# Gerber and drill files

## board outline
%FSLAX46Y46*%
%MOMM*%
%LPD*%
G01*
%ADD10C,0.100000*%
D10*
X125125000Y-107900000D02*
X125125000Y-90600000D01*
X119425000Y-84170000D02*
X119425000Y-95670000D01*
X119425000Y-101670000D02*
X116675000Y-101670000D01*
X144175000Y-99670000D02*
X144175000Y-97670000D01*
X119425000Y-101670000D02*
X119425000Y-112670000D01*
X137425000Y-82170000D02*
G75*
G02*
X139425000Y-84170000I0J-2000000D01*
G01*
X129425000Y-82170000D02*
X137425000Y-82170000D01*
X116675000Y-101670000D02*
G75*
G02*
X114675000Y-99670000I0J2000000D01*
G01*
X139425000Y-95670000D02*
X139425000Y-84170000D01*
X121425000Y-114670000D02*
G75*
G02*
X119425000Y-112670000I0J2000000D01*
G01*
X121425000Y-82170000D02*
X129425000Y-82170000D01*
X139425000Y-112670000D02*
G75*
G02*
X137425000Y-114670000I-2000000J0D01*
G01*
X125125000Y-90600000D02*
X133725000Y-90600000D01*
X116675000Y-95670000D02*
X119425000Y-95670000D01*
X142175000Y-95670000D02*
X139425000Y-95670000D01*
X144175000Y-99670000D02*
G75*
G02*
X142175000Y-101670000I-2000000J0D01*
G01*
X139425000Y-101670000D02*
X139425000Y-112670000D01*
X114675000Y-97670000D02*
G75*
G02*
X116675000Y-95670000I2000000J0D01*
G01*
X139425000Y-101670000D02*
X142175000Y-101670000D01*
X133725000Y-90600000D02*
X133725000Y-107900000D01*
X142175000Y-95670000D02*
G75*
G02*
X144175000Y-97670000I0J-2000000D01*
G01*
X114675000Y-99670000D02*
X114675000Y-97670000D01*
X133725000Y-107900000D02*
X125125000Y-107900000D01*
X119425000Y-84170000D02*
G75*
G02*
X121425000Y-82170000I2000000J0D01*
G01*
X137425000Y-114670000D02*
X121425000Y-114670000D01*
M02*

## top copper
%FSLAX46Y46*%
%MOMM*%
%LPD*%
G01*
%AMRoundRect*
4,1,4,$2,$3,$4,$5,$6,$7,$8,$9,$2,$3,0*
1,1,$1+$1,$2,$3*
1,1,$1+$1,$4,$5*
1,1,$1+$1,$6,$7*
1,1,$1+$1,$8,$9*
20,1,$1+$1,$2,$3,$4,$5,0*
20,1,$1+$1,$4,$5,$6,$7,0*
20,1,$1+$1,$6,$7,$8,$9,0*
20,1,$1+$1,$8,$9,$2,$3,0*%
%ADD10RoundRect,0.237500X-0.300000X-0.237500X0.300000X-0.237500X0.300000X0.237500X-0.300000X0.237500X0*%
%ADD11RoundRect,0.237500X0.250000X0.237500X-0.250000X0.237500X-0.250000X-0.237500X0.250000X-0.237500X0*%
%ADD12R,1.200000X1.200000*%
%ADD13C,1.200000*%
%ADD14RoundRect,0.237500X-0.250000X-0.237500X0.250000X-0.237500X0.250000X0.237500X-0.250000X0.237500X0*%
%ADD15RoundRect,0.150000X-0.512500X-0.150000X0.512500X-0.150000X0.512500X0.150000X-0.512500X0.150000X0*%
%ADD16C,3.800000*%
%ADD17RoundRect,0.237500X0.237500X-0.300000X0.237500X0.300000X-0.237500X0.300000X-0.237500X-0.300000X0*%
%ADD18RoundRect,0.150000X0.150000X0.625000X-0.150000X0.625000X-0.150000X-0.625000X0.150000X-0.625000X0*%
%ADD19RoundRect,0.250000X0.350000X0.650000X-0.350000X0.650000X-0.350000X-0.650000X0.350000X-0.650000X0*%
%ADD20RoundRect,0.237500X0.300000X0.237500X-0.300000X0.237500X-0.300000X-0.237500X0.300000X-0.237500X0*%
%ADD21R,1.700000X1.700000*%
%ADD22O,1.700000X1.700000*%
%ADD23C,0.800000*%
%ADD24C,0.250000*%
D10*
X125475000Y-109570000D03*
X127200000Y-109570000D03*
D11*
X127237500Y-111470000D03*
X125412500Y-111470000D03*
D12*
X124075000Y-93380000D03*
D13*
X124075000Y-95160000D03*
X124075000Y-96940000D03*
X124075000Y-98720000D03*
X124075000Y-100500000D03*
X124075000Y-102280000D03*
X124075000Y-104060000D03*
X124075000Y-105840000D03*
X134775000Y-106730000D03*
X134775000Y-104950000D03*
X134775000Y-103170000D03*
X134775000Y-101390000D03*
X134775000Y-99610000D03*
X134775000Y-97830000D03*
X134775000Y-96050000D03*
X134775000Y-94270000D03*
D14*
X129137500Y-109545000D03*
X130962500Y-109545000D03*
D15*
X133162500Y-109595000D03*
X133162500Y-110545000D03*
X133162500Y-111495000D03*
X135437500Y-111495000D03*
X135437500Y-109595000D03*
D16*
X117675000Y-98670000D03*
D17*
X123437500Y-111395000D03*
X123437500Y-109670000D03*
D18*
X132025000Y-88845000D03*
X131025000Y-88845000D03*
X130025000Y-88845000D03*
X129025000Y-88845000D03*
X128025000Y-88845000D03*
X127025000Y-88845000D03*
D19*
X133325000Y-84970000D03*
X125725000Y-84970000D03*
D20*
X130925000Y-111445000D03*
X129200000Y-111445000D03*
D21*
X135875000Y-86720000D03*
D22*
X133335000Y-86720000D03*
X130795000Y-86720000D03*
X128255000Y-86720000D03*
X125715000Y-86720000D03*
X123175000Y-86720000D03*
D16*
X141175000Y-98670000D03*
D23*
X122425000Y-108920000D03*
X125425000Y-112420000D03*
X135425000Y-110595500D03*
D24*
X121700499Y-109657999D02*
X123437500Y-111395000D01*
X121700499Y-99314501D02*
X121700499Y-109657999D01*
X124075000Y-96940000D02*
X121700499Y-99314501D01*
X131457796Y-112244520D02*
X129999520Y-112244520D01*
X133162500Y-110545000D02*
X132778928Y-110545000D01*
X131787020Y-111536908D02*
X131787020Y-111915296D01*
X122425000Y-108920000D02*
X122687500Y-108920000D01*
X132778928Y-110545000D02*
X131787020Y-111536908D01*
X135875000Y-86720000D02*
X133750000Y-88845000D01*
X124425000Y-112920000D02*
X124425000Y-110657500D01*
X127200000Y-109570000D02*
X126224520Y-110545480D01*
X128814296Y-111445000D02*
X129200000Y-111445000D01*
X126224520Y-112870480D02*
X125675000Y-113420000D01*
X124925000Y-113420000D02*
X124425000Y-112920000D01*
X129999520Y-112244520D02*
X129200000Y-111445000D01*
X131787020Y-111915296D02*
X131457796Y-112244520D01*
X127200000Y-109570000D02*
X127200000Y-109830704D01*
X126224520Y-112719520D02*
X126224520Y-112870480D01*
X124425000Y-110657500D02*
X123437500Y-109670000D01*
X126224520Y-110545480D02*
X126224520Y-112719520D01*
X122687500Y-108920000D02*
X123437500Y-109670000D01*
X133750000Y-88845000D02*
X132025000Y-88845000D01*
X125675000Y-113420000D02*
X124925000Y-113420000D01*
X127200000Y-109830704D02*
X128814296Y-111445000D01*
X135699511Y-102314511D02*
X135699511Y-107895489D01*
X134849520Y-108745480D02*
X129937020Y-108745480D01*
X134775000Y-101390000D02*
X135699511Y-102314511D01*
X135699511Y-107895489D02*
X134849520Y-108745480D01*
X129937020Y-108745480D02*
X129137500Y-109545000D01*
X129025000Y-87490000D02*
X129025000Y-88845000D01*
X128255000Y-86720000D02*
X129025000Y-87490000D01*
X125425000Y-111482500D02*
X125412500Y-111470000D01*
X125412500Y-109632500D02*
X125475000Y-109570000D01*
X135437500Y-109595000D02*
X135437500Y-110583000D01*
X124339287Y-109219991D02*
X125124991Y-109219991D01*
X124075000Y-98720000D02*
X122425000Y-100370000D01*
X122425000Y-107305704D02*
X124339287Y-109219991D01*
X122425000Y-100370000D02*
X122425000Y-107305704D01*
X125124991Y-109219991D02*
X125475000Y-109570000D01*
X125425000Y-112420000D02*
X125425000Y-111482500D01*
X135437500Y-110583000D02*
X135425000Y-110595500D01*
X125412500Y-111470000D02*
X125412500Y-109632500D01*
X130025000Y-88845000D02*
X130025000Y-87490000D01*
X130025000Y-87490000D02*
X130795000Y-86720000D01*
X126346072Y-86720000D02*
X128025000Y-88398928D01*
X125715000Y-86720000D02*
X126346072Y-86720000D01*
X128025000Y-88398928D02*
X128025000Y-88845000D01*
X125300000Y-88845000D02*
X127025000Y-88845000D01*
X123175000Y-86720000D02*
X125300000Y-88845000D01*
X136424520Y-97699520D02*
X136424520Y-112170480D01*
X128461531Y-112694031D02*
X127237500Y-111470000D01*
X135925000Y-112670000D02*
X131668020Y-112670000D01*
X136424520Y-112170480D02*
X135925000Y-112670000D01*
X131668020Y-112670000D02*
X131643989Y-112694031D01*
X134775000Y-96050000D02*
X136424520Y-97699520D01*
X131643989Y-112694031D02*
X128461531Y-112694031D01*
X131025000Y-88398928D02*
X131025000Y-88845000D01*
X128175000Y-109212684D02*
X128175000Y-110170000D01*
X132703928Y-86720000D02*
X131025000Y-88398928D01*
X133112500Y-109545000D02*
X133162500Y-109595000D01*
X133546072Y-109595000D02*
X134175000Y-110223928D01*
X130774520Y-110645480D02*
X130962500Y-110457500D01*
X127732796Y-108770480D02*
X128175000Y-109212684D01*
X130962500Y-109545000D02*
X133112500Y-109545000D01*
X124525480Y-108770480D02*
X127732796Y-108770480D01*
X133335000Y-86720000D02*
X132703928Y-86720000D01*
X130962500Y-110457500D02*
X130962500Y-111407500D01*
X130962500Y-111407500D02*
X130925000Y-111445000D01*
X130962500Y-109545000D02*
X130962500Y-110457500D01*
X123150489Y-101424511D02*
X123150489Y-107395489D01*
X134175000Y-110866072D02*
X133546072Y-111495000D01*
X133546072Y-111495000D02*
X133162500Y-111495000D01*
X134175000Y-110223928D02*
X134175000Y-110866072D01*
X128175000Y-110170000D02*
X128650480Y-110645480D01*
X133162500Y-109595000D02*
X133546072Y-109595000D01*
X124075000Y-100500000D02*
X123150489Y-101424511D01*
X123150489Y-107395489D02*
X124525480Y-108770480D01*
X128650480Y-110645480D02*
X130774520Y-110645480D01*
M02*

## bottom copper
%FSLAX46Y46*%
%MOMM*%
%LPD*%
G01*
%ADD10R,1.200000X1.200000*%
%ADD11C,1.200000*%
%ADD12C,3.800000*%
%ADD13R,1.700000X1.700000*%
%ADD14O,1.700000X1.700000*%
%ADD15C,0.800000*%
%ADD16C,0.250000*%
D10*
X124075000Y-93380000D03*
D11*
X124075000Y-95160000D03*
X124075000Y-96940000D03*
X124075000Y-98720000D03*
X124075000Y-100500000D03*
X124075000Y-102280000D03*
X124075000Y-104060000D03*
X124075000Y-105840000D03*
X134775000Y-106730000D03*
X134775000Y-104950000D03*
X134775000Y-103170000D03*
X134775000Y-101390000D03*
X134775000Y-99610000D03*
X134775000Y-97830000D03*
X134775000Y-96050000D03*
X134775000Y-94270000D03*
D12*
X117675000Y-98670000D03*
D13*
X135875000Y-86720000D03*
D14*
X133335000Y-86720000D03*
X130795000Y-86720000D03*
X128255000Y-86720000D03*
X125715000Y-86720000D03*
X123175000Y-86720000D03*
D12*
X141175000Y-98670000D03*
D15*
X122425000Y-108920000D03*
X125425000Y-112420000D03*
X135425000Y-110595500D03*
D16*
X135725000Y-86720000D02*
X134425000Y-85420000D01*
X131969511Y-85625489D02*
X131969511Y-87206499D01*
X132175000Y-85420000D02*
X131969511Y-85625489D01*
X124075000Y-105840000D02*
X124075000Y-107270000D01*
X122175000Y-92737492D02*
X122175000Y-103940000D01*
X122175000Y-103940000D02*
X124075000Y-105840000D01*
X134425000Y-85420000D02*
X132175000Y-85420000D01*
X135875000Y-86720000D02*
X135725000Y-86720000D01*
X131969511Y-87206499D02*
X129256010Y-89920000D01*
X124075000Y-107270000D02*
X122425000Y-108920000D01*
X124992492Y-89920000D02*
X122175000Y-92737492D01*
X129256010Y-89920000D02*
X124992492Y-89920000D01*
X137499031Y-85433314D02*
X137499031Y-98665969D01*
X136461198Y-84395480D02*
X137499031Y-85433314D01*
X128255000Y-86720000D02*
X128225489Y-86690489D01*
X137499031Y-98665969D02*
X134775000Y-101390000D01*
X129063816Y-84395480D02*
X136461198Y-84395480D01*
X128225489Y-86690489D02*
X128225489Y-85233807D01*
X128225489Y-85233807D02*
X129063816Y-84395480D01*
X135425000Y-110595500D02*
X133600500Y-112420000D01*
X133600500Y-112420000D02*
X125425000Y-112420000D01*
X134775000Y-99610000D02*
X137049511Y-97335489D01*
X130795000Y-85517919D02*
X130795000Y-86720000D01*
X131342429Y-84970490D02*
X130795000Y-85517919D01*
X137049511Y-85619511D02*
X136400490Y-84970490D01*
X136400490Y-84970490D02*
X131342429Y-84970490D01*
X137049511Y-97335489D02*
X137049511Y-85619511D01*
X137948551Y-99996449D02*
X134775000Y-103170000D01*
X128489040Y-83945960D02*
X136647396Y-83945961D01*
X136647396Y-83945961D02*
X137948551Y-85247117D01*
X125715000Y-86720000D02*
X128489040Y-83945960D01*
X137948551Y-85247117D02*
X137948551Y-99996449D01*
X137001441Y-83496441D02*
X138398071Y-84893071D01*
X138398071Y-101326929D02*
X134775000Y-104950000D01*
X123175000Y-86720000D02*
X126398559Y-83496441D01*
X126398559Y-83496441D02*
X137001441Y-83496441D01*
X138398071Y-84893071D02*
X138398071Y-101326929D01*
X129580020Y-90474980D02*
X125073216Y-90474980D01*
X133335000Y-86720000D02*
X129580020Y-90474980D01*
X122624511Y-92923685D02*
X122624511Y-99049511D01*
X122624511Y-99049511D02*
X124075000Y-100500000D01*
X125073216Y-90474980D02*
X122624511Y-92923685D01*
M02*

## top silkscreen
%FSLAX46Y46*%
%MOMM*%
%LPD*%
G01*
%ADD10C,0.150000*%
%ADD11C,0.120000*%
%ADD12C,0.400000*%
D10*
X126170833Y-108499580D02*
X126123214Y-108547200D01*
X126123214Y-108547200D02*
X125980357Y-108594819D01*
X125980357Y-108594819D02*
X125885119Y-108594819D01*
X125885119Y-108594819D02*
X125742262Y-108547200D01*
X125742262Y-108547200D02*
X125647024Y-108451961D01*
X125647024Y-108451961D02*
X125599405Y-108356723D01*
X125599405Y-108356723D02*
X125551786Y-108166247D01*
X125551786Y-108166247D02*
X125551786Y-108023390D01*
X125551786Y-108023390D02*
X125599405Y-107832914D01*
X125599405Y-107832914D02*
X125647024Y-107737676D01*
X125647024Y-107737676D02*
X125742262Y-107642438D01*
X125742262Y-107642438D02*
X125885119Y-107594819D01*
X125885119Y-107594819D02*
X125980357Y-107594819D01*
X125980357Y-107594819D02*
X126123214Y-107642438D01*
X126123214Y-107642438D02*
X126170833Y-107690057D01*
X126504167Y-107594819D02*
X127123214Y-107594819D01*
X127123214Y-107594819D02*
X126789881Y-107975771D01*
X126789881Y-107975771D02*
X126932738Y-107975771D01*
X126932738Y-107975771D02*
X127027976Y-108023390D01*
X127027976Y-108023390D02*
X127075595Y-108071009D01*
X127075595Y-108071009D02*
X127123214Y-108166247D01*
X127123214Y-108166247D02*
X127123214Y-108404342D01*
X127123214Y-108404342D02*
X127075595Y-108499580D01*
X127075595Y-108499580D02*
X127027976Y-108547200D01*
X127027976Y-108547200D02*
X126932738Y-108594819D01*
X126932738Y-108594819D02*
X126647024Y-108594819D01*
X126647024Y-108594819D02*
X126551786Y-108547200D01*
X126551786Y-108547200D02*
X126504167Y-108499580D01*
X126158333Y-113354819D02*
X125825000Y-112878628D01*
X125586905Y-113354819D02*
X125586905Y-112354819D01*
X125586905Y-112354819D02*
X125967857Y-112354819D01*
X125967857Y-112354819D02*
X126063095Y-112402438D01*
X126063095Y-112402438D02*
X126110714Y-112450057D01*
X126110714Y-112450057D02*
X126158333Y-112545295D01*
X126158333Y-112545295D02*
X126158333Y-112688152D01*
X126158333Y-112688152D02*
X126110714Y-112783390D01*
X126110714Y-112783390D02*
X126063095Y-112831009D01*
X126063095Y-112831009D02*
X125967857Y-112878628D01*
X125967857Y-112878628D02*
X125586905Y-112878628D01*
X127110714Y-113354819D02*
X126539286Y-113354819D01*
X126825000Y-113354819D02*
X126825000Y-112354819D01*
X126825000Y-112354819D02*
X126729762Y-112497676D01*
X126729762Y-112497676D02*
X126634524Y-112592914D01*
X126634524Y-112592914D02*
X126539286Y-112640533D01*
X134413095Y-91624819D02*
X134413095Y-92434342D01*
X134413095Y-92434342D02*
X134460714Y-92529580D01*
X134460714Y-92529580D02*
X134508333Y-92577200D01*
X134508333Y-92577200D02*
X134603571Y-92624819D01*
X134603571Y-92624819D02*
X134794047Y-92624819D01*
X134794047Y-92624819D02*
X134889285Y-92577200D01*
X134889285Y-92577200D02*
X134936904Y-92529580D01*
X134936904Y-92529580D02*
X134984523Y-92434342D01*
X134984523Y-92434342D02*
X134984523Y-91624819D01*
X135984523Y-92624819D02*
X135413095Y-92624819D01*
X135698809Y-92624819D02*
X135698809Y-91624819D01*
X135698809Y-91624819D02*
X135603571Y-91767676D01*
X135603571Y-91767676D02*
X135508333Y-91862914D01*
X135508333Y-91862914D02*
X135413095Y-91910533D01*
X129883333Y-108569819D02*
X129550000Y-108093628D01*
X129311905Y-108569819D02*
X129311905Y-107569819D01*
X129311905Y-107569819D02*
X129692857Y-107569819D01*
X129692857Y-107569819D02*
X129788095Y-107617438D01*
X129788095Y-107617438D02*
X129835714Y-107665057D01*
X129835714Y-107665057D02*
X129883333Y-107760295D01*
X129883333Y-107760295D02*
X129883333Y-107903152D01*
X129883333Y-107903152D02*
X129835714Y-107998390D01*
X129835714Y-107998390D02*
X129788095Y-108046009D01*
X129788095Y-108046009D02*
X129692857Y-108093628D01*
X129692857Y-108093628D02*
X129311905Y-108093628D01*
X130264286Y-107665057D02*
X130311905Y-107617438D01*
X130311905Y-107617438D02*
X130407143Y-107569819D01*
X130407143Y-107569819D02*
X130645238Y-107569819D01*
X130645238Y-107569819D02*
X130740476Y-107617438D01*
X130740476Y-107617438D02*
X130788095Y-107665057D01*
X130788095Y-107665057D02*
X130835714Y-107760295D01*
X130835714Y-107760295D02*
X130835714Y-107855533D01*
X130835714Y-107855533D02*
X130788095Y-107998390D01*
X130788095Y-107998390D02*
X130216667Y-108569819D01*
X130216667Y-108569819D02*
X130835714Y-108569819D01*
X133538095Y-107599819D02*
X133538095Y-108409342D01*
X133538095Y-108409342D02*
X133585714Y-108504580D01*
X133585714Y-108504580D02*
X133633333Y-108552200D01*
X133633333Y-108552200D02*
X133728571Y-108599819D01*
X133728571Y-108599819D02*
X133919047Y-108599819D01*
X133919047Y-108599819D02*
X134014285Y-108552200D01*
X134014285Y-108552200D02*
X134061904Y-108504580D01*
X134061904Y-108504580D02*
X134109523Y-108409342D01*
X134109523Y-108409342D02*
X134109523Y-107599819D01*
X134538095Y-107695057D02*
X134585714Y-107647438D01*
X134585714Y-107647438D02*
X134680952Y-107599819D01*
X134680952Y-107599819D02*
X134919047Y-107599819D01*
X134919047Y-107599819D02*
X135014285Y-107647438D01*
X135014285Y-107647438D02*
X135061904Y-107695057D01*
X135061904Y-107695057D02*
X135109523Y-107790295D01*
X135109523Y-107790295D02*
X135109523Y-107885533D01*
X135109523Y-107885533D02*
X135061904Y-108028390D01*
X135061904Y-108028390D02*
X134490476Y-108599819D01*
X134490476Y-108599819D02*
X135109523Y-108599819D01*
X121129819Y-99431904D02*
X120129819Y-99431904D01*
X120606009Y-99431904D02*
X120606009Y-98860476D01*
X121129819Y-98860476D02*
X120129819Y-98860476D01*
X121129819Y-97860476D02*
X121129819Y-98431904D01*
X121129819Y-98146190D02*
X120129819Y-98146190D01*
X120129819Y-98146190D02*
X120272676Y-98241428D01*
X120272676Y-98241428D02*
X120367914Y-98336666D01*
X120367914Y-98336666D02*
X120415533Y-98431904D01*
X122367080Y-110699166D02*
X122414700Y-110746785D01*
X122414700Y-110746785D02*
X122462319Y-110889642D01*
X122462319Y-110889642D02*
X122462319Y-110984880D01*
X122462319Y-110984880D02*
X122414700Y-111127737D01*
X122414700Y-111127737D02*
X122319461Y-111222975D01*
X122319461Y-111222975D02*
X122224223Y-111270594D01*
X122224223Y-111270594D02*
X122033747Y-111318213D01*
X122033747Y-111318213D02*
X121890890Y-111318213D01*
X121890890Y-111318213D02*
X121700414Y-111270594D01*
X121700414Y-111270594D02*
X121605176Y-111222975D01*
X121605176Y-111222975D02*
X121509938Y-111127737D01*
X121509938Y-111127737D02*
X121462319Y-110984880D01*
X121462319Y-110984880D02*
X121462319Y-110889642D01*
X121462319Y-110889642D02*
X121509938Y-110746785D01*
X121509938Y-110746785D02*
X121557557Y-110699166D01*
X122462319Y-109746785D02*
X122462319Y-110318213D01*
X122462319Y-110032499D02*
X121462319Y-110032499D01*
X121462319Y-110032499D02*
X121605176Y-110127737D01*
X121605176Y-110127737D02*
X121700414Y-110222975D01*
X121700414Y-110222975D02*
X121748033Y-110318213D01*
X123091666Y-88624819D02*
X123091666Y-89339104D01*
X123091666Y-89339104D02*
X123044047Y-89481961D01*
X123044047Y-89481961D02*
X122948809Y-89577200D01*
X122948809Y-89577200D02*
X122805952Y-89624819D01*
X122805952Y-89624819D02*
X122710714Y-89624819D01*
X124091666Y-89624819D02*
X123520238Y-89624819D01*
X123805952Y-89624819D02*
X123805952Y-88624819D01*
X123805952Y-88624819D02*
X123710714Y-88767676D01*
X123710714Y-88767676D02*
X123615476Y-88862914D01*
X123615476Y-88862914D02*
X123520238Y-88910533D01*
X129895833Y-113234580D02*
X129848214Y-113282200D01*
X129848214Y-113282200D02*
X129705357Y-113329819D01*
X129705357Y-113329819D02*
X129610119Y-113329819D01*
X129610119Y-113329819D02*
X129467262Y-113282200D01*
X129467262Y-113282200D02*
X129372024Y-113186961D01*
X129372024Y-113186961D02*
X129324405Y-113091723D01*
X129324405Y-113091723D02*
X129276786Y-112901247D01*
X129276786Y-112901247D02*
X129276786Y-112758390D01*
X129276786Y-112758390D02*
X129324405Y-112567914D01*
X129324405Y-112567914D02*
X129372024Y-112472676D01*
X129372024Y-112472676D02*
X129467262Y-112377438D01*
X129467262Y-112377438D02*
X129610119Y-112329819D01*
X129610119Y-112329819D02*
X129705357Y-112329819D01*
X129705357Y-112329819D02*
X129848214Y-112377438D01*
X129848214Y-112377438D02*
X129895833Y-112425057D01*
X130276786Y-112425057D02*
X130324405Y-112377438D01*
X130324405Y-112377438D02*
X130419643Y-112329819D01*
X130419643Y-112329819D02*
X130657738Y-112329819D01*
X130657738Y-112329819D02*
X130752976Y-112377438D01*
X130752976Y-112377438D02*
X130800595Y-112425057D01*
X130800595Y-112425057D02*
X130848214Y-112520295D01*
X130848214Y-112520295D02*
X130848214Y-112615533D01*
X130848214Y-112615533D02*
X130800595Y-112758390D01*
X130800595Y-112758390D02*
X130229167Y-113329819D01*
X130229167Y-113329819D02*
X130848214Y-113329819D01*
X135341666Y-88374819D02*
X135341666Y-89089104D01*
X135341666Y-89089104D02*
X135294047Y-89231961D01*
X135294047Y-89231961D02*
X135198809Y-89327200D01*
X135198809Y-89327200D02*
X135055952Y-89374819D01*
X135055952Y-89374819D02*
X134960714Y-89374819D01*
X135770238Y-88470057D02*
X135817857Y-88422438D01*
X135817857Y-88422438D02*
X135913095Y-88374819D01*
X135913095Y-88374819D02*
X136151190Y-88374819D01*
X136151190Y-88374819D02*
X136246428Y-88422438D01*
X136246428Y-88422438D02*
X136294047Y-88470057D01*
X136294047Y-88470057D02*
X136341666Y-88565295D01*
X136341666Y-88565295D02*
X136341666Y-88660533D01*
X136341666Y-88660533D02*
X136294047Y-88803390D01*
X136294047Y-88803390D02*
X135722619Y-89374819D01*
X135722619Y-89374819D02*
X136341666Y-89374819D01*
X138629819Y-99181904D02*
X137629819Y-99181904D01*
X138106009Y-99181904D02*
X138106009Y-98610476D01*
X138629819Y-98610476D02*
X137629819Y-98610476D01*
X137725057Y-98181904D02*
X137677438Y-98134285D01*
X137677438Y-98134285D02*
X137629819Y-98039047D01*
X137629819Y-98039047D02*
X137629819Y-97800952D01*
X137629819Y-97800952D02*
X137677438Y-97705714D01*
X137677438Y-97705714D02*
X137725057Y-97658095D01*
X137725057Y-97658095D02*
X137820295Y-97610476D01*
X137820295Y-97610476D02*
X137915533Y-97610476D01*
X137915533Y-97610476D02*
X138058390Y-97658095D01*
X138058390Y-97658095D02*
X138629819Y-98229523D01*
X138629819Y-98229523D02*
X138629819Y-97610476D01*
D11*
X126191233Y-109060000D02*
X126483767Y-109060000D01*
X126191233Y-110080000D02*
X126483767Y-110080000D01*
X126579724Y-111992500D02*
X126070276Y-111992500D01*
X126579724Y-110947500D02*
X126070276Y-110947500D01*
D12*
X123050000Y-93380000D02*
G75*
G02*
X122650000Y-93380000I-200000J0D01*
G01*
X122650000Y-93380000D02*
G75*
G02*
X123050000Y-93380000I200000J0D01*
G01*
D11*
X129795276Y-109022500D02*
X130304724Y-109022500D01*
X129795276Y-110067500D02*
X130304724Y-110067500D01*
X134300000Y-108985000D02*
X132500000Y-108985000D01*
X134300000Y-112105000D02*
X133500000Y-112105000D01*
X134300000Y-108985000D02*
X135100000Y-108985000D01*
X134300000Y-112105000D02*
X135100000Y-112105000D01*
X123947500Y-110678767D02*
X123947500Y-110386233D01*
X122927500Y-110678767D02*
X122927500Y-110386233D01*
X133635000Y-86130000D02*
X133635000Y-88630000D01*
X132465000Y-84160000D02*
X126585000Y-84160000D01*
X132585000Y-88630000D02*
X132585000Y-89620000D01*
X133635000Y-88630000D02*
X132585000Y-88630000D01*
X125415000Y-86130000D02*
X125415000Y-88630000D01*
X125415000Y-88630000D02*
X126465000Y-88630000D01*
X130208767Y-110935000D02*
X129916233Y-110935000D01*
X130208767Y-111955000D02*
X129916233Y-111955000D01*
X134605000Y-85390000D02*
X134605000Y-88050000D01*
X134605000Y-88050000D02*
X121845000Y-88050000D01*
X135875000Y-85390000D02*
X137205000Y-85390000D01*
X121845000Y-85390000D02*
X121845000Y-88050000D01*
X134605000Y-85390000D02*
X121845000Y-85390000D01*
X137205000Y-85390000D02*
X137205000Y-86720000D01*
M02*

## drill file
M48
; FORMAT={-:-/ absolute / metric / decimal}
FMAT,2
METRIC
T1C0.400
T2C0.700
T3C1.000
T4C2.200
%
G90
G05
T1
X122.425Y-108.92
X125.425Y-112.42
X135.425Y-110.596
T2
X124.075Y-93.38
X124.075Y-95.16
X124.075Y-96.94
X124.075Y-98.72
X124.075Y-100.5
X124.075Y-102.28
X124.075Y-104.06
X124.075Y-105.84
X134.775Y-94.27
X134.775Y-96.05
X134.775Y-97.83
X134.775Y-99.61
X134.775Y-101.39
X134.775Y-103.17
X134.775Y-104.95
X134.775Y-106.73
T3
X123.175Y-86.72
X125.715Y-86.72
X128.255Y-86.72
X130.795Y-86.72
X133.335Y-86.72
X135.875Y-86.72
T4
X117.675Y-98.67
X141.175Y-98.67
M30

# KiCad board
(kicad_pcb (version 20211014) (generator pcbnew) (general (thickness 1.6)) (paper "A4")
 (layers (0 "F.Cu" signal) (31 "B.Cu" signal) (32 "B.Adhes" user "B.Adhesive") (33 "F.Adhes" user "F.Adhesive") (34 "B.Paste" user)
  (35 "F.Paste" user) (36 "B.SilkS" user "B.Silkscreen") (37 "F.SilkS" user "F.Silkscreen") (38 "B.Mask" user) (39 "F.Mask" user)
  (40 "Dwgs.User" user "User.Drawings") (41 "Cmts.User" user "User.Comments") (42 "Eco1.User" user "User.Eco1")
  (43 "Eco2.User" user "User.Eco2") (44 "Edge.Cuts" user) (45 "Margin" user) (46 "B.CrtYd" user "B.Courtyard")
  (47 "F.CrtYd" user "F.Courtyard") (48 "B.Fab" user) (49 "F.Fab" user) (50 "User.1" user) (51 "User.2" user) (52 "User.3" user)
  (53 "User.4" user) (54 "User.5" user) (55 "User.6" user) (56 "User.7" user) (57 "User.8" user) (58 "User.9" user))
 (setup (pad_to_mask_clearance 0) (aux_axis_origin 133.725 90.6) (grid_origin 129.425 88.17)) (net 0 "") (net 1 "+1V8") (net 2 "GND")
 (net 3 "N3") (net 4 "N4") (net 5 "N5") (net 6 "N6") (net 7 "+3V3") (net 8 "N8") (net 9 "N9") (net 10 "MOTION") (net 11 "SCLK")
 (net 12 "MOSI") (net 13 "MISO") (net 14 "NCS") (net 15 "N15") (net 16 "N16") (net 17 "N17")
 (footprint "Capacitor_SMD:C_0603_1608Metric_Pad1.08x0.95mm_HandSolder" (layer "F.Cu") (at 126.3375 109.57)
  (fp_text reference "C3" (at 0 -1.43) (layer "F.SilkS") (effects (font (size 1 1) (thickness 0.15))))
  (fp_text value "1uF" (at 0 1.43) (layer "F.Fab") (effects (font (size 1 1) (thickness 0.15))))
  (fp_line (start -0.146267 -0.51) (end 0.146267 -0.51) (layer "F.SilkS") (width 0.12))
  (fp_line (start -0.146267 0.51) (end 0.146267 0.51) (layer "F.SilkS") (width 0.12))
  (pad "1" smd roundrect (at -0.8625 0) (size 1.075 0.95) (layers "F.Cu" "F.Paste" "F.Mask") (roundrect_rratio 0.25) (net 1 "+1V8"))
  (pad "2" smd roundrect (at 0.8625 0) (size 1.075 0.95) (layers "F.Cu" "F.Paste" "F.Mask") (roundrect_rratio 0.25) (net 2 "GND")))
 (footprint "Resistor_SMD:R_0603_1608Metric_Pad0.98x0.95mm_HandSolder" (layer "F.Cu") (at 126.325 111.47 180)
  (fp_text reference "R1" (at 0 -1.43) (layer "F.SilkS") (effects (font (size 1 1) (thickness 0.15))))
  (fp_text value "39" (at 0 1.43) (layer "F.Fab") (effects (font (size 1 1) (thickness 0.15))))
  (fp_line (start -0.254724 -0.5225) (end 0.254724 -0.5225) (layer "F.SilkS") (width 0.12))
  (fp_line (start -0.254724 0.5225) (end 0.254724 0.5225) (layer "F.SilkS") (width 0.12))
  (pad "1" smd roundrect (at -0.9125 0 180) (size 0.975 0.95) (layers "F.Cu" "F.Paste" "F.Mask") (roundrect_rratio 0.25) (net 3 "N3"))
  (pad "2" smd roundrect (at 0.9125 0 180) (size 0.975 0.95) (layers "F.Cu" "F.Paste" "F.Mask") (roundrect_rratio 0.25) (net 1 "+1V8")))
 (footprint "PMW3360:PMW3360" (layer "F.Cu") (at 124.075 93.38)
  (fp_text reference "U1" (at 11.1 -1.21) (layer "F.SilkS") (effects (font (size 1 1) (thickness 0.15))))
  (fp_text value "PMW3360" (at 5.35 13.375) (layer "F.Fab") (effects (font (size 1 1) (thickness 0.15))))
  (fp_circle (center -1.225 0) (end -1.025 0) (layer "F.SilkS") (width 0.4) (fill none))
  (pad "1" thru_hole rect (at 0 0) (size 1.2 1.2) (drill 0.7) (layers *.Cu *.Mask) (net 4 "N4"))
  (pad "2" thru_hole circle (at 0 1.78) (size 1.2 1.2) (drill 0.7) (layers *.Cu *.Mask) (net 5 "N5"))
  (pad "3" thru_hole circle (at 0 3.56) (size 1.2 1.2) (drill 0.7) (layers *.Cu *.Mask) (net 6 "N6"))
  (pad "4" thru_hole circle (at 0 5.34) (size 1.2 1.2) (drill 0.7) (layers *.Cu *.Mask) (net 1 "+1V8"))
  (pad "5" thru_hole circle (at 0 7.12) (size 1.2 1.2) (drill 0.7) (layers *.Cu *.Mask) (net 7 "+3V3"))
  (pad "6" thru_hole circle (at 0 8.9) (size 1.2 1.2) (drill 0.7) (layers *.Cu *.Mask) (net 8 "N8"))
  (pad "7" thru_hole circle (at 0 10.68) (size 1.2 1.2) (drill 0.7) (layers *.Cu *.Mask) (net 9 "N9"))
  (pad "8" thru_hole circle (at 0 12.46) (size 1.2 1.2) (drill 0.7) (layers *.Cu *.Mask) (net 2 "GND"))
  (pad "9" thru_hole circle (at 10.7 13.35) (size 1.2 1.2) (drill 0.7) (layers *.Cu *.Mask) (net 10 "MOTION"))
  (pad "10" thru_hole circle (at 10.7 11.57) (size 1.2 1.2) (drill 0.7) (layers *.Cu *.Mask) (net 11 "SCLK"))
  (pad "11" thru_hole circle (at 10.7 9.79) (size 1.2 1.2) (drill 0.7) (layers *.Cu *.Mask) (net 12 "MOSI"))
  (pad "12" thru_hole circle (at 10.7 8.01) (size 1.2 1.2) (drill 0.7) (layers *.Cu *.Mask) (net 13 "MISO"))
  (pad "13" thru_hole circle (at 10.7 6.23) (size 1.2 1.2) (drill 0.7) (layers *.Cu *.Mask) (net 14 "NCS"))
  (pad "14" thru_hole circle (at 10.7 4.45) (size 1.2 1.2) (drill 0.7) (layers *.Cu *.Mask) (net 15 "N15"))
  (pad "15" thru_hole circle (at 10.7 2.67) (size 1.2 1.2) (drill 0.7) (layers *.Cu *.Mask) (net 3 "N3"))
  (pad "16" thru_hole circle (at 10.7 0.89) (size 1.2 1.2) (drill 0.7) (layers *.Cu *.Mask) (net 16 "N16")))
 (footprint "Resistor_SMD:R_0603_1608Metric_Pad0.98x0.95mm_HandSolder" (layer "F.Cu") (at 130.05 109.545)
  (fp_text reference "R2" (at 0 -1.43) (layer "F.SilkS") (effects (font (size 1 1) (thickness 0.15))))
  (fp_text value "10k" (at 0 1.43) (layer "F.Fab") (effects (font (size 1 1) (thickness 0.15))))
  (fp_line (start -0.254724 -0.5225) (end 0.254724 -0.5225) (layer "F.SilkS") (width 0.12))
  (fp_line (start -0.254724 0.5225) (end 0.254724 0.5225) (layer "F.SilkS") (width 0.12))
  (pad "1" smd roundrect (at -0.9125 0) (size 0.975 0.95) (layers "F.Cu" "F.Paste" "F.Mask") (roundrect_rratio 0.25) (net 13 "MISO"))
  (pad "2" smd roundrect (at 0.9125 0) (size 0.975 0.95) (layers "F.Cu" "F.Paste" "F.Mask") (roundrect_rratio 0.25) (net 7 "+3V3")))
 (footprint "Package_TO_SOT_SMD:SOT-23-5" (layer "F.Cu") (at 134.3 110.545)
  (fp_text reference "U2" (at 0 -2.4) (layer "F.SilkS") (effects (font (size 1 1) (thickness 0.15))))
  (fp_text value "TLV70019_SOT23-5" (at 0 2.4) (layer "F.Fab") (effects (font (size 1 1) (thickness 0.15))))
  (fp_line (start 0 -1.56) (end -1.8 -1.56) (layer "F.SilkS") (width 0.12))
  (fp_line (start 0 1.56) (end -0.8 1.56) (layer "F.SilkS") (width 0.12))
  (fp_line (start 0 -1.56) (end 0.8 -1.56) (layer "F.SilkS") (width 0.12))
  (fp_line (start 0 1.56) (end 0.8 1.56) (layer "F.SilkS") (width 0.12))
  (pad "1" smd roundrect (at -1.1375 -0.95) (size 1.325 0.6) (layers "F.Cu" "F.Paste" "F.Mask") (roundrect_rratio 0.25) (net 7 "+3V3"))
  (pad "2" smd roundrect (at -1.1375 0) (size 1.325 0.6) (layers "F.Cu" "F.Paste" "F.Mask") (roundrect_rratio 0.25) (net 2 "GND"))
  (pad "3" smd roundrect (at -1.1375 0.95) (size 1.325 0.6) (layers "F.Cu" "F.Paste" "F.Mask") (roundrect_rratio 0.25) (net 7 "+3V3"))
  (pad "4" smd roundrect (at 1.1375 0.95) (size 1.325 0.6) (layers "F.Cu" "F.Paste" "F.Mask") (roundrect_rratio 0.25) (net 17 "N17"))
  (pad "5" smd roundrect (at 1.1375 -0.95) (size 1.325 0.6) (layers "F.Cu" "F.Paste" "F.Mask") (roundrect_rratio 0.25) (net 1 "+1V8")))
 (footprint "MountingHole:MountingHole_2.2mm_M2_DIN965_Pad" (layer "F.Cu") (at 117.675 98.67)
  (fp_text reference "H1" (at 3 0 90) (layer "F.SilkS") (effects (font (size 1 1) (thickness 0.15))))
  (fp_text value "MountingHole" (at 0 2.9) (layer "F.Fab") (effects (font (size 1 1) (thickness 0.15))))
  (pad "1" thru_hole circle (at 0 0) (size 3.8 3.8) (drill 2.2) (layers *.Cu *.Mask)))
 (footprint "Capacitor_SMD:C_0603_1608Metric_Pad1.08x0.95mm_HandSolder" (layer "F.Cu") (at 123.4375 110.5325 90)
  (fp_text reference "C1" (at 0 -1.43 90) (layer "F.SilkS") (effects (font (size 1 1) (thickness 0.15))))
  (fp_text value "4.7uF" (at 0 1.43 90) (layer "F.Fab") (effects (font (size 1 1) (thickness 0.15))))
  (fp_line (start -0.146267 0.51) (end 0.146267 0.51) (layer "F.SilkS") (width 0.12))
  (fp_line (start -0.146267 -0.51) (end 0.146267 -0.51) (layer "F.SilkS") (width 0.12))
  (pad "1" smd roundrect (at -0.8625 0 90) (size 1.075 0.95) (layers "F.Cu" "F.Paste" "F.Mask") (roundrect_rratio 0.25) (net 6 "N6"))
  (pad "2" smd roundrect (at 0.8625 0 90) (size 1.075 0.95) (layers "F.Cu" "F.Paste" "F.Mask") (roundrect_rratio 0.25) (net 2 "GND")))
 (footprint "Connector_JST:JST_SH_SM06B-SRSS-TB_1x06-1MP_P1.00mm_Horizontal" (layer "F.Cu") (at 129.525 86.845 180)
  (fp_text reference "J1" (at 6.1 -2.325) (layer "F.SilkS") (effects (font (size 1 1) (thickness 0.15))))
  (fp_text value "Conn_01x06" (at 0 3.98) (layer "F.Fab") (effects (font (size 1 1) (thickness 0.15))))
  (fp_line (start -4.11 0.715) (end -4.11 -1.785) (layer "F.SilkS") (width 0.12))
  (fp_line (start -2.94 2.685) (end 2.94 2.685) (layer "F.SilkS") (width 0.12))
  (fp_line (start -3.06 -1.785) (end -3.06 -2.775) (layer "F.SilkS") (width 0.12))
  (fp_line (start -4.11 -1.785) (end -3.06 -1.785) (layer "F.SilkS") (width 0.12))
  (fp_line (start 4.11 0.715) (end 4.11 -1.785) (layer "F.SilkS") (width 0.12))
  (fp_line (start 4.11 -1.785) (end 3.06 -1.785) (layer "F.SilkS") (width 0.12))
  (pad "1" smd roundrect (at -2.5 -2 180) (size 0.6 1.55) (layers "F.Cu" "F.Paste" "F.Mask") (roundrect_rratio 0.25) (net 2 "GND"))
  (pad "2" smd roundrect (at -1.5 -2 180) (size 0.6 1.55) (layers "F.Cu" "F.Paste" "F.Mask") (roundrect_rratio 0.25) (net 7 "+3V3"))
  (pad "3" smd roundrect (at -0.5 -2 180) (size 0.6 1.55) (layers "F.Cu" "F.Paste" "F.Mask") (roundrect_rratio 0.25) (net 14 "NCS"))
  (pad "4" smd roundrect (at 0.5 -2 180) (size 0.6 1.55) (layers "F.Cu" "F.Paste" "F.Mask") (roundrect_rratio 0.25) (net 13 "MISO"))
  (pad "5" smd roundrect (at 1.5 -2 180) (size 0.6 1.55) (layers "F.Cu" "F.Paste" "F.Mask") (roundrect_rratio 0.25) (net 12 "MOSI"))
  (pad "6" smd roundrect (at 2.5 -2 180) (size 0.6 1.55) (layers "F.Cu" "F.Paste" "F.Mask") (roundrect_rratio 0.25) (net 11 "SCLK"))
  (pad "MP" smd roundrect (at -3.8 1.875 180) (size 1.2 1.8) (layers "F.Cu" "F.Paste" "F.Mask") (roundrect_rratio 0.2083333333))
  (pad "MP" smd roundrect (at 3.8 1.875 180) (size 1.2 1.8) (layers "F.Cu" "F.Paste" "F.Mask") (roundrect_rratio 0.2083333333)))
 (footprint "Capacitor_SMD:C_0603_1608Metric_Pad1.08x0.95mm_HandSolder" (layer "F.Cu") (at 130.0625 111.445 180)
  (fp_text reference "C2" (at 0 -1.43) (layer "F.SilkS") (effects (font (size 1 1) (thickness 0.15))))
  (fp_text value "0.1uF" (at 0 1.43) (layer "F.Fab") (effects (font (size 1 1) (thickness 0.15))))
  (fp_line (start -0.146267 0.51) (end 0.146267 0.51) (layer "F.SilkS") (width 0.12))
  (fp_line (start -0.146267 -0.51) (end 0.146267 -0.51) (layer "F.SilkS") (width 0.12))
  (pad "1" smd roundrect (at -0.8625 0 180) (size 1.075 0.95) (layers "F.Cu" "F.Paste" "F.Mask") (roundrect_rratio 0.25) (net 7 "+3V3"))
  (pad "2" smd roundrect (at 0.8625 0 180) (size 1.075 0.95) (layers "F.Cu" "F.Paste" "F.Mask") (roundrect_rratio 0.25) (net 2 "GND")))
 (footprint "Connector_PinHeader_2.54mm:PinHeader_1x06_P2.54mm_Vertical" (layer "F.Cu") (at 135.875 86.72 -90)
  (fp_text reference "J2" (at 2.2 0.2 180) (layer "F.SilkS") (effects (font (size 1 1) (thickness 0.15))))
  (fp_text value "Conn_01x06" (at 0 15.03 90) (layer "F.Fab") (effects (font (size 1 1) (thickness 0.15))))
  (fp_line (start -1.33 1.27) (end 1.33 1.27) (layer "F.SilkS") (width 0.12))
  (fp_line (start 1.33 1.27) (end 1.33 14.03) (layer "F.SilkS") (width 0.12))
  (fp_line (start -1.33 0) (end -1.33 -1.33) (layer "F.SilkS") (width 0.12))
  (fp_line (start -1.33 14.03) (end 1.33 14.03) (layer "F.SilkS") (width 0.12))
  (fp_line (start -1.33 1.27) (end -1.33 14.03) (layer "F.SilkS") (width 0.12))
  (fp_line (start -1.33 -1.33) (end 0 -1.33) (layer "F.SilkS") (width 0.12))
  (pad "1" thru_hole rect (at 0 0 270) (size 1.7 1.7) (drill 1) (layers *.Cu *.Mask) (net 2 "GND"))
  (pad "2" thru_hole oval (at 0 2.54 270) (size 1.7 1.7) (drill 1) (layers *.Cu *.Mask) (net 7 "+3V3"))
  (pad "3" thru_hole oval (at 0 5.08 270) (size 1.7 1.7) (drill 1) (layers *.Cu *.Mask) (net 14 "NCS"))
  (pad "4" thru_hole oval (at 0 7.62 270) (size 1.7 1.7) (drill 1) (layers *.Cu *.Mask) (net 13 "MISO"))
  (pad "5" thru_hole oval (at 0 10.16 270) (size 1.7 1.7) (drill 1) (layers *.Cu *.Mask) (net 12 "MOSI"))
  (pad "6" thru_hole oval (at 0 12.7 270) (size 1.7 1.7) (drill 1) (layers *.Cu *.Mask) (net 11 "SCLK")))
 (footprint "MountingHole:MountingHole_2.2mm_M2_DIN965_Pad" (layer "F.Cu") (at 141.175 98.67)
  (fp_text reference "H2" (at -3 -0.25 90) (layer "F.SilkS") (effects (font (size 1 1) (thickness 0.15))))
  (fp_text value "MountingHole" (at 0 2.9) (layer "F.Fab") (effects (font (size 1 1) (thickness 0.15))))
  (pad "1" thru_hole circle (at 0 0) (size 3.8 3.8) (drill 2.2) (layers *.Cu *.Mask)))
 (gr_line (start 125.125 107.9) (end 125.125 90.6) (layer "Edge.Cuts") (width 0.1))
 (gr_line (start 119.425 84.17) (end 119.425 95.67) (layer "Edge.Cuts") (width 0.1))
 (gr_line (start 119.425 101.67) (end 116.675 101.67) (layer "Edge.Cuts") (width 0.1))
 (gr_line (start 144.175 99.67) (end 144.175 97.67) (layer "Edge.Cuts") (width 0.1))
 (gr_line (start 119.425 101.67) (end 119.425 112.67) (layer "Edge.Cuts") (width 0.1))
 (gr_arc (start 137.425 82.17) (mid 138.839214 82.755786) (end 139.425 84.17) (layer "Edge.Cuts") (width 0.1))
 (gr_line (start 129.425 82.17) (end 137.425 82.17) (layer "Edge.Cuts") (width 0.1))
 (gr_arc (start 116.675 101.67) (mid 115.260786 101.084214) (end 114.675 99.67) (layer "Edge.Cuts") (width 0.1))
 (gr_line (start 139.425 95.67) (end 139.425 84.17) (layer "Edge.Cuts") (width 0.1))
 (gr_arc (start 121.425 114.67) (mid 120.010786 114.084214) (end 119.425 112.67) (layer "Edge.Cuts") (width 0.1))
 (gr_line (start 121.425 82.17) (end 129.425 82.17) (layer "Edge.Cuts") (width 0.1))
 (gr_arc (start 139.425 112.67) (mid 138.839214 114.084214) (end 137.425 114.67) (layer "Edge.Cuts") (width 0.1))
 (gr_line (start 125.125 90.6) (end 133.725 90.6) (layer "Edge.Cuts") (width 0.1))
 (gr_line (start 116.675 95.67) (end 119.425 95.67) (layer "Edge.Cuts") (width 0.1))
 (gr_line (start 142.175 95.67) (end 139.425 95.67) (layer "Edge.Cuts") (width 0.1))
 (gr_arc (start 144.175 99.67) (mid 143.589214 101.084214) (end 142.175 101.67) (layer "Edge.Cuts") (width 0.1))
 (gr_line (start 139.425 101.67) (end 139.425 112.67) (layer "Edge.Cuts") (width 0.1))
 (gr_arc (start 114.675 97.67) (mid 115.260786 96.255786) (end 116.675 95.67) (layer "Edge.Cuts") (width 0.1))
 (gr_line (start 139.425 101.67) (end 142.175 101.67) (layer "Edge.Cuts") (width 0.1))
 (gr_line (start 133.725 90.6) (end 133.725 107.9) (layer "Edge.Cuts") (width 0.1))
 (gr_arc (start 142.175 95.67) (mid 143.589214 96.255786) (end 144.175 97.67) (layer "Edge.Cuts") (width 0.1))
 (gr_line (start 114.675 99.67) (end 114.675 97.67) (layer "Edge.Cuts") (width 0.1))
 (gr_line (start 133.725 107.9) (end 125.125 107.9) (layer "Edge.Cuts") (width 0.1))
 (gr_arc (start 119.425 84.17) (mid 120.010786 82.755786) (end 121.425 82.17) (layer "Edge.Cuts") (width 0.1))
 (gr_line (start 137.425 114.67) (end 121.425 114.67) (layer "Edge.Cuts") (width 0.1))
 (segment (start 121.700499 109.657999) (end 123.4375 111.395) (width 0.25) (layer "F.Cu") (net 6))
 (segment (start 121.700499 99.314501) (end 121.700499 109.657999) (width 0.25) (layer "F.Cu") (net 6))
 (segment (start 124.075 96.94) (end 121.700499 99.314501) (width 0.25) (layer "F.Cu") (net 6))
 (segment (start 131.457796 112.24452) (end 129.99952 112.24452) (width 0.25) (layer "F.Cu") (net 2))
 (segment (start 133.1625 110.545) (end 132.778928 110.545) (width 0.25) (layer "F.Cu") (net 2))
 (segment (start 131.78702 111.536908) (end 131.78702 111.915296) (width 0.25) (layer "F.Cu") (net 2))
 (segment (start 122.425 108.92) (end 122.6875 108.92) (width 0.25) (layer "F.Cu") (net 2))
 (segment (start 132.778928 110.545) (end 131.78702 111.536908) (width 0.25) (layer "F.Cu") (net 2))
 (segment (start 135.875 86.72) (end 133.75 88.845) (width 0.25) (layer "F.Cu") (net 2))
 (segment (start 124.425 112.92) (end 124.425 110.6575) (width 0.25) (layer "F.Cu") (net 2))
 (segment (start 127.2 109.57) (end 126.22452 110.54548) (width 0.25) (layer "F.Cu") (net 2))
 (segment (start 128.814296 111.445) (end 129.2 111.445) (width 0.25) (layer "F.Cu") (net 2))
 (segment (start 126.22452 112.87048) (end 125.675 113.42) (width 0.25) (layer "F.Cu") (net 2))
 (segment (start 124.925 113.42) (end 124.425 112.92) (width 0.25) (layer "F.Cu") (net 2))
 (segment (start 129.99952 112.24452) (end 129.2 111.445) (width 0.25) (layer "F.Cu") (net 2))
 (segment (start 131.78702 111.915296) (end 131.457796 112.24452) (width 0.25) (layer "F.Cu") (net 2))
 (segment (start 127.2 109.57) (end 127.2 109.830704) (width 0.25) (layer "F.Cu") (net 2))
 (segment (start 126.22452 112.71952) (end 126.22452 112.87048) (width 0.25) (layer "F.Cu") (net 2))
 (segment (start 124.425 110.6575) (end 123.4375 109.67) (width 0.25) (layer "F.Cu") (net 2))
 (segment (start 126.22452 110.54548) (end 126.22452 112.71952) (width 0.25) (layer "F.Cu") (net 2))
 (segment (start 122.6875 108.92) (end 123.4375 109.67) (width 0.25) (layer "F.Cu") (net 2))
 (segment (start 133.75 88.845) (end 132.025 88.845) (width 0.25) (layer "F.Cu") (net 2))
 (segment (start 125.675 113.42) (end 124.925 113.42) (width 0.25) (layer "F.Cu") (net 2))
 (segment (start 127.2 109.830704) (end 128.814296 111.445) (width 0.25) (layer "F.Cu") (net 2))
 (via (at 122.425 108.92) (size 0.8) (drill 0.4) (layers "F.Cu" "B.Cu") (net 2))
 (segment (start 135.725 86.72) (end 134.425 85.42) (width 0.25) (layer "B.Cu") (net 2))
 (segment (start 131.969511 85.625489) (end 131.969511 87.206499) (width 0.25) (layer "B.Cu") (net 2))
 (segment (start 132.175 85.42) (end 131.969511 85.625489) (width 0.25) (layer "B.Cu") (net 2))
 (segment (start 124.075 105.84) (end 124.075 107.27) (width 0.25) (layer "B.Cu") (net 2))
 (segment (start 122.175 92.737492) (end 122.175 103.94) (width 0.25) (layer "B.Cu") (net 2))
 (segment (start 122.175 103.94) (end 124.075 105.84) (width 0.25) (layer "B.Cu") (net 2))
 (segment (start 134.425 85.42) (end 132.175 85.42) (width 0.25) (layer "B.Cu") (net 2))
 (segment (start 135.875 86.72) (end 135.725 86.72) (width 0.25) (layer "B.Cu") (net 2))
 (segment (start 131.969511 87.206499) (end 129.25601 89.92) (width 0.25) (layer "B.Cu") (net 2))
 (segment (start 124.075 107.27) (end 122.425 108.92) (width 0.25) (layer "B.Cu") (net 2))
 (segment (start 124.992492 89.92) (end 122.175 92.737492) (width 0.25) (layer "B.Cu") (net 2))
 (segment (start 129.25601 89.92) (end 124.992492 89.92) (width 0.25) (layer "B.Cu") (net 2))
 (segment (start 135.699511 102.314511) (end 135.699511 107.895489) (width 0.25) (layer "F.Cu") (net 13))
 (segment (start 134.84952 108.74548) (end 129.93702 108.74548) (width 0.25) (layer "F.Cu") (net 13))
 (segment (start 134.775 101.39) (end 135.699511 102.314511) (width 0.25) (layer "F.Cu") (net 13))
 (segment (start 135.699511 107.895489) (end 134.84952 108.74548) (width 0.25) (layer "F.Cu") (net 13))
 (segment (start 129.93702 108.74548) (end 129.1375 109.545) (width 0.25) (layer "F.Cu") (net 13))
 (segment (start 129.025 87.49) (end 129.025 88.845) (width 0.25) (layer "F.Cu") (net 13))
 (segment (start 128.255 86.72) (end 129.025 87.49) (width 0.25) (layer "F.Cu") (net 13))
 (segment (start 137.499031 85.433314) (end 137.499031 98.665969) (width 0.25) (layer "B.Cu") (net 13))
 (segment (start 136.461198 84.39548) (end 137.499031 85.433314) (width 0.25) (layer "B.Cu") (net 13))
 (segment (start 128.255 86.72) (end 128.225489 86.690489) (width 0.25) (layer "B.Cu") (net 13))
 (segment (start 137.499031 98.665969) (end 134.775 101.39) (width 0.25) (layer "B.Cu") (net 13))
 (segment (start 129.063816 84.39548) (end 136.461198 84.39548) (width 0.25) (layer "B.Cu") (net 13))
 (segment (start 128.225489 86.690489) (end 128.225489 85.233807) (width 0.25) (layer "B.Cu") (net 13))
 (segment (start 128.225489 85.233807) (end 129.063816 84.39548) (width 0.25) (layer "B.Cu") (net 13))
 (segment (start 125.425 111.4825) (end 125.4125 111.47) (width 0.25) (layer "F.Cu") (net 1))
 (segment (start 125.4125 109.6325) (end 125.475 109.57) (width 0.25) (layer "F.Cu") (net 1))
 (segment (start 135.4375 109.595) (end 135.4375 110.583) (width 0.25) (layer "F.Cu") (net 1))
 (segment (start 124.339287 109.219991) (end 125.124991 109.219991) (width 0.25) (layer "F.Cu") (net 1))
 (segment (start 124.075 98.72) (end 122.425 100.37) (width 0.25) (layer "F.Cu") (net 1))
 (segment (start 122.425 107.305704) (end 124.339287 109.219991) (width 0.25) (layer "F.Cu") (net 1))
 (segment (start 122.425 100.37) (end 122.425 107.305704) (width 0.25) (layer "F.Cu") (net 1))
 (segment (start 125.124991 109.219991) (end 125.475 109.57) (width 0.25) (layer "F.Cu") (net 1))
 (segment (start 125.425 112.42) (end 125.425 111.4825) (width 0.25) (layer "F.Cu") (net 1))
 (segment (start 135.4375 110.583) (end 135.425 110.5955) (width 0.25) (layer "F.Cu") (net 1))
 (segment (start 125.4125 111.47) (end 125.4125 109.6325) (width 0.25) (layer "F.Cu") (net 1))
 (via (at 125.425 112.42) (size 0.8) (drill 0.4) (layers "F.Cu" "B.Cu") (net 1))
 (via (at 135.425 110.5955) (size 0.8) (drill 0.4) (layers "F.Cu" "B.Cu") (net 1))
 (segment (start 135.425 110.5955) (end 133.6005 112.42) (width 0.25) (layer "B.Cu") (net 1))
 (segment (start 133.6005 112.42) (end 125.425 112.42) (width 0.25) (layer "B.Cu") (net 1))
 (segment (start 130.025 88.845) (end 130.025 87.49) (width 0.25) (layer "F.Cu") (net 14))
 (segment (start 130.025 87.49) (end 130.795 86.72) (width 0.25) (layer "F.Cu") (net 14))
 (segment (start 134.775 99.61) (end 137.049511 97.335489) (width 0.25) (layer "B.Cu") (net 14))
 (segment (start 130.795 85.517919) (end 130.795 86.72) (width 0.25) (layer "B.Cu") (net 14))
 (segment (start 131.342429 84.97049) (end 130.795 85.517919) (width 0.25) (layer "B.Cu") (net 14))
 (segment (start 137.049511 85.619511) (end 136.40049 84.97049) (width 0.25) (layer "B.Cu") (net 14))
 (segment (start 136.40049 84.97049) (end 131.342429 84.97049) (width 0.25) (layer "B.Cu") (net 14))
 (segment (start 137.049511 97.335489) (end 137.049511 85.619511) (width 0.25) (layer "B.Cu") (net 14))
 (segment (start 126.346072 86.72) (end 128.025 88.398928) (width 0.25) (layer "F.Cu") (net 12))
 (segment (start 125.715 86.72) (end 126.346072 86.72) (width 0.25) (layer "F.Cu") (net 12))
 (segment (start 128.025 88.398928) (end 128.025 88.845) (width 0.25) (layer "F.Cu") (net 12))
 (segment (start 137.948551 99.996449) (end 134.775 103.17) (width 0.25) (layer "B.Cu") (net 12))
 (segment (start 128.48904 83.94596) (end 136.647396 83.945961) (width 0.25) (layer "B.Cu") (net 12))
 (segment (start 136.647396 83.945961) (end 137.948551 85.247117) (width 0.25) (layer "B.Cu") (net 12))
 (segment (start 125.715 86.72) (end 128.48904 83.94596) (width 0.25) (layer "B.Cu") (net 12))
 (segment (start 137.948551 85.247117) (end 137.948551 99.996449) (width 0.25) (layer "B.Cu") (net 12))
 (segment (start 125.3 88.845) (end 127.025 88.845) (width 0.25) (layer "F.Cu") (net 11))
 (segment (start 123.175 86.72) (end 125.3 88.845) (width 0.25) (layer "F.Cu") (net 11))
 (segment (start 137.001441 83.496441) (end 138.398071 84.893071) (width 0.25) (layer "B.Cu") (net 11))
 (segment (start 138.398071 101.326929) (end 134.775 104.95) (width 0.25) (layer "B.Cu") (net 11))
 (segment (start 123.175 86.72) (end 126.398559 83.496441) (width 0.25) (layer "B.Cu") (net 11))
 (segment (start 126.398559 83.496441) (end 137.001441 83.496441) (width 0.25) (layer "B.Cu") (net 11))
 (segment (start 138.398071 84.893071) (end 138.398071 101.326929) (width 0.25) (layer "B.Cu") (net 11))
 (segment (start 136.42452 97.69952) (end 136.42452 112.17048) (width 0.25) (layer "F.Cu") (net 3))
 (segment (start 128.461531 112.694031) (end 127.2375 111.47) (width 0.25) (layer "F.Cu") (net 3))
 (segment (start 135.925 112.67) (end 131.66802 112.67) (width 0.25) (layer "F.Cu") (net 3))
 (segment (start 136.42452 112.17048) (end 135.925 112.67) (width 0.25) (layer "F.Cu") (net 3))
 (segment (start 131.66802 112.67) (end 131.643989 112.694031) (width 0.25) (layer "F.Cu") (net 3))
 (segment (start 134.775 96.05) (end 136.42452 97.69952) (width 0.25) (layer "F.Cu") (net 3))
 (segment (start 131.643989 112.694031) (end 128.461531 112.694031) (width 0.25) (layer "F.Cu") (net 3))
 (segment (start 131.025 88.398928) (end 131.025 88.845) (width 0.25) (layer "F.Cu") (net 7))
 (segment (start 128.175 109.212684) (end 128.175 110.17) (width 0.25) (layer "F.Cu") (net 7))
 (segment (start 132.703928 86.72) (end 131.025 88.398928) (width 0.25) (layer "F.Cu") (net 7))
 (segment (start 133.1125 109.545) (end 133.1625 109.595) (width 0.25) (layer "F.Cu") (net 7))
 (segment (start 133.546072 109.595) (end 134.175 110.223928) (width 0.25) (layer "F.Cu") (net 7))
 (segment (start 130.77452 110.64548) (end 130.9625 110.4575) (width 0.25) (layer "F.Cu") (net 7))
 (segment (start 127.732796 108.77048) (end 128.175 109.212684) (width 0.25) (layer "F.Cu") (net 7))
 (segment (start 130.9625 109.545) (end 133.1125 109.545) (width 0.25) (layer "F.Cu") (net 7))
 (segment (start 124.52548 108.77048) (end 127.732796 108.77048) (width 0.25) (layer "F.Cu") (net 7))
 (segment (start 133.335 86.72) (end 132.703928 86.72) (width 0.25) (layer "F.Cu") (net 7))
 (segment (start 130.9625 110.4575) (end 130.9625 111.4075) (width 0.25) (layer "F.Cu") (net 7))
 (segment (start 130.9625 111.4075) (end 130.925 111.445) (width 0.25) (layer "F.Cu") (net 7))
 (segment (start 130.9625 109.545) (end 130.9625 110.4575) (width 0.25) (layer "F.Cu") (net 7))
 (segment (start 123.150489 101.424511) (end 123.150489 107.395489) (width 0.25) (layer "F.Cu") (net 7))
 (segment (start 134.175 110.866072) (end 133.546072 111.495) (width 0.25) (layer "F.Cu") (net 7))
 (segment (start 133.546072 111.495) (end 133.1625 111.495) (width 0.25) (layer "F.Cu") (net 7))
 (segment (start 134.175 110.223928) (end 134.175 110.866072) (width 0.25) (layer "F.Cu") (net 7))
 (segment (start 128.175 110.17) (end 128.65048 110.64548) (width 0.25) (layer "F.Cu") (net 7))
 (segment (start 133.1625 109.595) (end 133.546072 109.595) (width 0.25) (layer "F.Cu") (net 7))
 (segment (start 124.075 100.5) (end 123.150489 101.424511) (width 0.25) (layer "F.Cu") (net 7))
 (segment (start 123.150489 107.395489) (end 124.52548 108.77048) (width 0.25) (layer "F.Cu") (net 7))
 (segment (start 128.65048 110.64548) (end 130.77452 110.64548) (width 0.25) (layer "F.Cu") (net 7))
 (segment (start 129.58002 90.47498) (end 125.073216 90.47498) (width 0.25) (layer "B.Cu") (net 7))
 (segment (start 133.335 86.72) (end 129.58002 90.47498) (width 0.25) (layer "B.Cu") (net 7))
 (segment (start 122.624511 92.923685) (end 122.624511 99.049511) (width 0.25) (layer "B.Cu") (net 7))
 (segment (start 122.624511 99.049511) (end 124.075 100.5) (width 0.25) (layer "B.Cu") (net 7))
 (segment (start 125.073216 90.47498) (end 122.624511 92.923685) (width 0.25) (layer "B.Cu") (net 7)))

